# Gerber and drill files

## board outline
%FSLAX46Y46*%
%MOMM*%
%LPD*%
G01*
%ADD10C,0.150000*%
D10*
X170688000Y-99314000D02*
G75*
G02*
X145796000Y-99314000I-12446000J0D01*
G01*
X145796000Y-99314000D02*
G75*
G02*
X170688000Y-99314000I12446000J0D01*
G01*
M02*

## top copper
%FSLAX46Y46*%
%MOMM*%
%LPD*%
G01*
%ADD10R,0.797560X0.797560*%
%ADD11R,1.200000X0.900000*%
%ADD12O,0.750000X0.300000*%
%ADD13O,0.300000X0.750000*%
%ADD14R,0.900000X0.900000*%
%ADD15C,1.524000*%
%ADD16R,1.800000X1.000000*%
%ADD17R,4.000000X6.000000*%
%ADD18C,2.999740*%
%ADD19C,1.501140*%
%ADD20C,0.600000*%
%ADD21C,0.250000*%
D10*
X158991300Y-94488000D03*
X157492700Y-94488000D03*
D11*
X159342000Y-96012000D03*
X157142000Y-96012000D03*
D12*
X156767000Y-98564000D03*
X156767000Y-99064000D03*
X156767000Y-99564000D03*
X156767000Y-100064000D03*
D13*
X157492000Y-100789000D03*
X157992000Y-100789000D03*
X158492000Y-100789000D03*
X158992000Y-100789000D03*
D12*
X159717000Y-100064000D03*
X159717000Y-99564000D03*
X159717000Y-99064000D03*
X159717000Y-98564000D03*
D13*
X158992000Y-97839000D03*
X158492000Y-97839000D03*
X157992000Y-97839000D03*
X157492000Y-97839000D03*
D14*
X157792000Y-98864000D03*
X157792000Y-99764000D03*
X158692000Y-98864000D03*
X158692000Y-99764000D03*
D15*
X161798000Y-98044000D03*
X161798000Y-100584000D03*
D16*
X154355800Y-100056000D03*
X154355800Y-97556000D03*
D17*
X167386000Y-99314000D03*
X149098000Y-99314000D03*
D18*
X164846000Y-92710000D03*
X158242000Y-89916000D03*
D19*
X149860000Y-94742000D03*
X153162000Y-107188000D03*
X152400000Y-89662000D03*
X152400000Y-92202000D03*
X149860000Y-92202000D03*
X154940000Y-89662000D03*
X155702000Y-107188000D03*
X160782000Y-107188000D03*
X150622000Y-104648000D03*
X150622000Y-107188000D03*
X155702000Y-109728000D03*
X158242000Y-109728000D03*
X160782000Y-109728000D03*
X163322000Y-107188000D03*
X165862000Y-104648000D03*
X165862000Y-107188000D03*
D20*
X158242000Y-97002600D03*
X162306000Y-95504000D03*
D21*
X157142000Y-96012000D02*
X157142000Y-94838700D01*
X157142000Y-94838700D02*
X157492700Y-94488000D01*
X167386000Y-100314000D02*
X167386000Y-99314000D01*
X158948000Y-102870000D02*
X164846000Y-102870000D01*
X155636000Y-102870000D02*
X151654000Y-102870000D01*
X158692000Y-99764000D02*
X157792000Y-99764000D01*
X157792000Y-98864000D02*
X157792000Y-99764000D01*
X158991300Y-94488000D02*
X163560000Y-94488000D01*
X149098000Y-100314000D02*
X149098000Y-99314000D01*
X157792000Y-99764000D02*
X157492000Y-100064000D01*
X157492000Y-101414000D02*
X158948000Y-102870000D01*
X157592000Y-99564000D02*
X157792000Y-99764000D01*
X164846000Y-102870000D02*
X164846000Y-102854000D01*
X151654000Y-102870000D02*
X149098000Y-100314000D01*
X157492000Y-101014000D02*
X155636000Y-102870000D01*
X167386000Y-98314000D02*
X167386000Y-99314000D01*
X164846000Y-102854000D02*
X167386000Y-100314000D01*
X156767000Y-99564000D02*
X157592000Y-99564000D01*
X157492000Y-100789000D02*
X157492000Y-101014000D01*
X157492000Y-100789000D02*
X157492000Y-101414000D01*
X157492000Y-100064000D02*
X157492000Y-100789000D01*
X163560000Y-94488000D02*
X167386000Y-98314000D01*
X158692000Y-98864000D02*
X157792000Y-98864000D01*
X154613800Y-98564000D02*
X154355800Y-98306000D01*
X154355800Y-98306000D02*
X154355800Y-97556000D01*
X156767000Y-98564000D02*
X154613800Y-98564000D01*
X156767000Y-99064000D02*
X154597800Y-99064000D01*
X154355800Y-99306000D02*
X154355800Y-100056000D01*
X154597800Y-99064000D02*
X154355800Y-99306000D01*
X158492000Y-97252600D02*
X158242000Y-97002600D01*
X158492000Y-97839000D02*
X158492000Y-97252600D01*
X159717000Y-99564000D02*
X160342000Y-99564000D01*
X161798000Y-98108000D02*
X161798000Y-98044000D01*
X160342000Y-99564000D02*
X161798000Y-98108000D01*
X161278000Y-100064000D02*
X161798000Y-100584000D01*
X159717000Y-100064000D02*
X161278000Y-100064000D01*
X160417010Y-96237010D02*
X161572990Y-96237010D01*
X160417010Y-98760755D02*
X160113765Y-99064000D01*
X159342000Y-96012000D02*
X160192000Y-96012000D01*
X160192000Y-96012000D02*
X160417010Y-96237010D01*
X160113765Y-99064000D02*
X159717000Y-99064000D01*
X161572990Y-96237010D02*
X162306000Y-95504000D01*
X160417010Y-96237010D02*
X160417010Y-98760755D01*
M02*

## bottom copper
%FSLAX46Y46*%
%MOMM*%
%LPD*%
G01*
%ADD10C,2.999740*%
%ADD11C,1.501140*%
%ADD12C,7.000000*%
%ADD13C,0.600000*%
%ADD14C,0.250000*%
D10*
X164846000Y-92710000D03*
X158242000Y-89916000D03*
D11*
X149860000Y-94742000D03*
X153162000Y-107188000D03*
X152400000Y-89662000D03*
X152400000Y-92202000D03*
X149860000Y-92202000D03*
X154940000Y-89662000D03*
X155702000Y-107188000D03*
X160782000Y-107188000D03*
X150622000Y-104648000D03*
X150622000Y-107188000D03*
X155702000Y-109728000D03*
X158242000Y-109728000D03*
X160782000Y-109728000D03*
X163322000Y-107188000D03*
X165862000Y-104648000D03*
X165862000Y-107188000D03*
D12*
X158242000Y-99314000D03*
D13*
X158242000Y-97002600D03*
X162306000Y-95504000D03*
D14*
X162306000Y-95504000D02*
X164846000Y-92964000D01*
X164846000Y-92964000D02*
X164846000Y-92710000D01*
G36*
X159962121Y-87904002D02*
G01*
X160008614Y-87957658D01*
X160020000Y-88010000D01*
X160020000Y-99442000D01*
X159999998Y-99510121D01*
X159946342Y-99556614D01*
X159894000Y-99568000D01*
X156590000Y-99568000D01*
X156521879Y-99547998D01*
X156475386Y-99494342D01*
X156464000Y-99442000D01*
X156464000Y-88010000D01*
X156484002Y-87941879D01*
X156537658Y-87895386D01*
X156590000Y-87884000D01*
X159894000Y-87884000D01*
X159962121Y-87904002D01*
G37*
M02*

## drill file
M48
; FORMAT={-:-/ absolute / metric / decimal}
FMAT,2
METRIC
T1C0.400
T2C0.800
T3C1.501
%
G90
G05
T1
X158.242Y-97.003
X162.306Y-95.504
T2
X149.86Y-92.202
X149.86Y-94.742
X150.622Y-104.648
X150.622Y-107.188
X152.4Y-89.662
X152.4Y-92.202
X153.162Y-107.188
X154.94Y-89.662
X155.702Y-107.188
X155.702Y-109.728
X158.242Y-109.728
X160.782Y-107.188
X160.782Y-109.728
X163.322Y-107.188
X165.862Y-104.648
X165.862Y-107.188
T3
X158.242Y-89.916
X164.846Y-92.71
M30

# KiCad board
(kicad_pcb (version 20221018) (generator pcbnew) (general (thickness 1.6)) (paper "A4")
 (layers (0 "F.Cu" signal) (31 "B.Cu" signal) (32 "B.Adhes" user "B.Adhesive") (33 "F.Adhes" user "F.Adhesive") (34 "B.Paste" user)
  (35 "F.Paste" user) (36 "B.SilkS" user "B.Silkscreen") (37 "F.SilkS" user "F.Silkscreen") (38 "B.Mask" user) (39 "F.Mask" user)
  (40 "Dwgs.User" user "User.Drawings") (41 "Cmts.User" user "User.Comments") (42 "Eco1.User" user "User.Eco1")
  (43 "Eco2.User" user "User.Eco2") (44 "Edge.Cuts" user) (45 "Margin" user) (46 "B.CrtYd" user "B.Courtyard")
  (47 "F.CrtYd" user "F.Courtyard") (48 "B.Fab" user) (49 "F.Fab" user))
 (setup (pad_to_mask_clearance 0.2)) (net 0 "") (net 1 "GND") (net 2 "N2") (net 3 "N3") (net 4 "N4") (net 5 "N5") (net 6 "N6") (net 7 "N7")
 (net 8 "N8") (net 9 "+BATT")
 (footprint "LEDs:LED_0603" (layer "F.Cu") (at 158.242 94.488 180)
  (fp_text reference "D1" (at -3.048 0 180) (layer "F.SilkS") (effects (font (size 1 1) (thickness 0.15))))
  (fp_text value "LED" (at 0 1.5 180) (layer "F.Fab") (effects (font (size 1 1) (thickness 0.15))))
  (pad "1" smd rect (at -0.7493 0) (size 0.79756 0.79756) (layers "F.Cu" "F.Paste" "F.Mask") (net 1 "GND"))
  (pad "2" smd rect (at 0.7493 0) (size 0.79756 0.79756) (layers "F.Cu" "F.Paste" "F.Mask") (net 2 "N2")))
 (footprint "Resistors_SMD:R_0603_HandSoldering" (layer "F.Cu") (at 158.242 96.012 180)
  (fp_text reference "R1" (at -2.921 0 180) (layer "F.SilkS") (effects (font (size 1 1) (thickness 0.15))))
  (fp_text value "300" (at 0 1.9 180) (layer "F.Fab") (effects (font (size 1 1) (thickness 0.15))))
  (pad "1" smd rect (at -1.1 0 180) (size 1.2 0.9) (layers "F.Cu" "F.Paste" "F.Mask") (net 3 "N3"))
  (pad "2" smd rect (at 1.1 0 180) (size 1.2 0.9) (layers "F.Cu" "F.Paste" "F.Mask") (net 2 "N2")))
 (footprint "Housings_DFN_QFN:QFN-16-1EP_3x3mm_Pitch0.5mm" (layer "F.Cu") (at 158.242 99.314)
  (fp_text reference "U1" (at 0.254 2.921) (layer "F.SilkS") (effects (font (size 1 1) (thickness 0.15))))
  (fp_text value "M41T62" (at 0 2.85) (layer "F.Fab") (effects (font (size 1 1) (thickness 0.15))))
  (pad "1" smd oval (at -1.475 -0.75) (size 0.75 0.3) (layers "F.Cu" "F.Paste" "F.Mask") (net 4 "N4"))
  (pad "2" smd oval (at -1.475 -0.25) (size 0.75 0.3) (layers "F.Cu" "F.Paste" "F.Mask") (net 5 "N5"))
  (pad "3" smd oval (at -1.475 0.25) (size 0.75 0.3) (layers "F.Cu" "F.Paste" "F.Mask") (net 1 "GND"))
  (pad "4" smd oval (at -1.475 0.75) (size 0.75 0.3) (layers "F.Cu" "F.Paste" "F.Mask") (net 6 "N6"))
  (pad "5" smd oval (at -0.75 1.475 90) (size 0.75 0.3) (layers "F.Cu" "F.Paste" "F.Mask") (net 1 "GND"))
  (pad "6" smd oval (at -0.25 1.475 90) (size 0.75 0.3) (layers "F.Cu" "F.Paste" "F.Mask"))
  (pad "7" smd oval (at 0.25 1.475 90) (size 0.75 0.3) (layers "F.Cu" "F.Paste" "F.Mask"))
  (pad "8" smd oval (at 0.75 1.475 90) (size 0.75 0.3) (layers "F.Cu" "F.Paste" "F.Mask"))
  (pad "9" smd oval (at 1.475 0.75) (size 0.75 0.3) (layers "F.Cu" "F.Paste" "F.Mask") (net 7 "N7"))
  (pad "10" smd oval (at 1.475 0.25) (size 0.75 0.3) (layers "F.Cu" "F.Paste" "F.Mask") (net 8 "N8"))
  (pad "11" smd oval (at 1.475 -0.25) (size 0.75 0.3) (layers "F.Cu" "F.Paste" "F.Mask") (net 3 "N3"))
  (pad "12" smd oval (at 1.475 -0.75) (size 0.75 0.3) (layers "F.Cu" "F.Paste" "F.Mask"))
  (pad "13" smd oval (at 0.75 -1.475 90) (size 0.75 0.3) (layers "F.Cu" "F.Paste" "F.Mask"))
  (pad "14" smd oval (at 0.25 -1.475 90) (size 0.75 0.3) (layers "F.Cu" "F.Paste" "F.Mask") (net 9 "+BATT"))
  (pad "15" smd oval (at -0.25 -1.475 90) (size 0.75 0.3) (layers "F.Cu" "F.Paste" "F.Mask"))
  (pad "16" smd oval (at -0.75 -1.475 90) (size 0.75 0.3) (layers "F.Cu" "F.Paste" "F.Mask"))
  (pad "17" smd rect (at -0.45 -0.45) (size 0.9 0.9) (layers "F.Cu" "F.Paste" "F.Mask") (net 1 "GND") (solder_paste_margin_ratio -0.2))
  (pad "17" smd rect (at -0.45 0.45) (size 0.9 0.9) (layers "F.Cu" "F.Paste" "F.Mask") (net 1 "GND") (solder_paste_margin_ratio -0.2))
  (pad "17" smd rect (at 0.45 -0.45) (size 0.9 0.9) (layers "F.Cu" "F.Paste" "F.Mask") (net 1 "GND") (solder_paste_margin_ratio -0.2))
  (pad "17" smd rect (at 0.45 0.45) (size 0.9 0.9) (layers "F.Cu" "F.Paste" "F.Mask") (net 1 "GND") (solder_paste_margin_ratio -0.2)))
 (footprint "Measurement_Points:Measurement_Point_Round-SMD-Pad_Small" (layer "F.Cu") (at 161.798 98.044)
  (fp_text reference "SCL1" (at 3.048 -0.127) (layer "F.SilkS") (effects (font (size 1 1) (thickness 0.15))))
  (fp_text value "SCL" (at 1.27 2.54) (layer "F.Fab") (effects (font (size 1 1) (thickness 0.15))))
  (pad "1" smd circle (at 0 0) (size 1.524 1.524) (layers "F.Cu" "F.Mask") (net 8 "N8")))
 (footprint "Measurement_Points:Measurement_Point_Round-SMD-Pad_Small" (layer "F.Cu") (at 161.798 100.584)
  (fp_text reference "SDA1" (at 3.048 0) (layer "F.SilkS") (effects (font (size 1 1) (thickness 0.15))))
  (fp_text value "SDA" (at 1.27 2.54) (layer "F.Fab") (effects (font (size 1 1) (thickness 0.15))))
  (pad "1" smd circle (at 0 0) (size 1.524 1.524) (layers "F.Cu" "F.Mask") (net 7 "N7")))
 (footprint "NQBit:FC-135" (layer "F.Cu") (at 154.3558 98.806 -90)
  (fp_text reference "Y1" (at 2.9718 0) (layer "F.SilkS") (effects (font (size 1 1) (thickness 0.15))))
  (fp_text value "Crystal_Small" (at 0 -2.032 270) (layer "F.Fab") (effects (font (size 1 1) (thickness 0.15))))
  (pad "1" smd rect (at 1.25 0 270) (size 1 1.8) (layers "F.Cu" "F.Paste" "F.Mask") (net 5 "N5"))
  (pad "2" smd rect (at -1.25 0 270) (size 1 1.8) (layers "F.Cu" "F.Paste" "F.Mask") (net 4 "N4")))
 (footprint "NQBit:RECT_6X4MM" (layer "F.Cu") (at 167.386 99.314)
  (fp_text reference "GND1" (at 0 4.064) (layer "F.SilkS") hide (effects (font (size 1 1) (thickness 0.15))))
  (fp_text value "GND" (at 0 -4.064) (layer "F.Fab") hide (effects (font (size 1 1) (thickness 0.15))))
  (pad "1" smd rect (at 0 0) (size 4 6) (layers "F.Cu" "F.Paste" "F.Mask") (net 1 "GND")))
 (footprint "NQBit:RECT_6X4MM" (layer "F.Cu") (at 149.098 99.314)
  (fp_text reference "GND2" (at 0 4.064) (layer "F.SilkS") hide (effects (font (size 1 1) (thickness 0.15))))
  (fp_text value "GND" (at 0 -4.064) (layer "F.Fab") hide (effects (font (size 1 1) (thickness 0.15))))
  (pad "1" smd rect (at 0 0) (size 4 6) (layers "F.Cu" "F.Paste" "F.Mask") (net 1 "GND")))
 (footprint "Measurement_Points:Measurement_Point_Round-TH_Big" (layer "F.Cu") (at 164.846 92.71)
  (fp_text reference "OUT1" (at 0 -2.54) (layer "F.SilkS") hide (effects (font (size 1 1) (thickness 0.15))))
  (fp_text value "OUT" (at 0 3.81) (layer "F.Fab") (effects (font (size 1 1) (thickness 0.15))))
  (pad "1" thru_hole circle (at 0 0) (size 2.99974 2.99974) (drill 1.50114) (layers "*.Cu" "*.Mask" "F.SilkS") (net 3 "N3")))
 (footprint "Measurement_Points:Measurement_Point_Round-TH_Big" (layer "F.Cu") (at 158.242 89.916)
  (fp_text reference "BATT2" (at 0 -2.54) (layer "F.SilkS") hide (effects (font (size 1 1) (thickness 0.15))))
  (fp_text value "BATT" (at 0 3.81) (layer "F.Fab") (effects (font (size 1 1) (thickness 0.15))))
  (pad "1" thru_hole circle (at 0 0) (size 2.99974 2.99974) (drill 1.50114) (layers "*.Cu" "*.Mask" "F.SilkS") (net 9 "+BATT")))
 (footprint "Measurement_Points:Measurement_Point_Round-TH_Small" (layer "F.Cu") (at 149.86 94.742)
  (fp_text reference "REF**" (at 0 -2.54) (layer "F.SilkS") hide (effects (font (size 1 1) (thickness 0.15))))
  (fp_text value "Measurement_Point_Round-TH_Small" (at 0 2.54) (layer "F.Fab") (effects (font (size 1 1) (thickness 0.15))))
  (pad "1" thru_hole circle (at 0 0) (size 1.50114 1.50114) (drill 0.8001) (layers "*.Cu" "*.Mask" "F.SilkS")))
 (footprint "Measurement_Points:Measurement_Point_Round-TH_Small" (layer "F.Cu") (at 153.162 107.188)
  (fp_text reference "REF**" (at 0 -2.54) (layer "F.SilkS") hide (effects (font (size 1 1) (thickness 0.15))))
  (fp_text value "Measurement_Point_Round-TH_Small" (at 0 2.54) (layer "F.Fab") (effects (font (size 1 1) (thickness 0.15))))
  (pad "1" thru_hole circle (at 0 0) (size 1.50114 1.50114) (drill 0.8001) (layers "*.Cu" "*.Mask" "F.SilkS")))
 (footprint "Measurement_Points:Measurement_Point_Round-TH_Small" (layer "F.Cu") (at 152.4 89.662)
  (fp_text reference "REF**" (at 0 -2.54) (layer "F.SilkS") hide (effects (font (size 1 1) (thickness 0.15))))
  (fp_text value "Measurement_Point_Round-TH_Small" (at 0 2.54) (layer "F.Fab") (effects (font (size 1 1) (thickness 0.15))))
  (pad "1" thru_hole circle (at 0 0) (size 1.50114 1.50114) (drill 0.8001) (layers "*.Cu" "*.Mask" "F.SilkS")))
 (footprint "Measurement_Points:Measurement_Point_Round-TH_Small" (layer "F.Cu") (at 152.4 92.202)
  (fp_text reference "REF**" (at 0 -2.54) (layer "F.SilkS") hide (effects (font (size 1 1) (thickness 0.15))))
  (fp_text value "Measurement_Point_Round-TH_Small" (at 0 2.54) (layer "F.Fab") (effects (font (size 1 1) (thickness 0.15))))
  (pad "1" thru_hole circle (at 0 0) (size 1.50114 1.50114) (drill 0.8001) (layers "*.Cu" "*.Mask" "F.SilkS")))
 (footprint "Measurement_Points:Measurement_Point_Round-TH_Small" (layer "F.Cu") (at 149.86 92.202)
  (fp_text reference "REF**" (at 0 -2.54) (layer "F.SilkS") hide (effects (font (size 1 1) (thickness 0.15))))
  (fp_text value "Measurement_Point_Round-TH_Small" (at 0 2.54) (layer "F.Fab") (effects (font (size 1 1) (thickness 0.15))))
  (pad "1" thru_hole circle (at 0 0) (size 1.50114 1.50114) (drill 0.8001) (layers "*.Cu" "*.Mask" "F.SilkS")))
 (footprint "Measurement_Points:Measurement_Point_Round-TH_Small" (layer "F.Cu") (at 154.94 89.662)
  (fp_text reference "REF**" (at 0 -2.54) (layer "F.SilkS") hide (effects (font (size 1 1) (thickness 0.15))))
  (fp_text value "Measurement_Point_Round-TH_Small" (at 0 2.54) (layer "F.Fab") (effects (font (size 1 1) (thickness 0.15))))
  (pad "1" thru_hole circle (at 0 0) (size 1.50114 1.50114) (drill 0.8001) (layers "*.Cu" "*.Mask" "F.SilkS")))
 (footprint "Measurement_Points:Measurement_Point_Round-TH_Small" (layer "F.Cu") (at 155.702 107.188)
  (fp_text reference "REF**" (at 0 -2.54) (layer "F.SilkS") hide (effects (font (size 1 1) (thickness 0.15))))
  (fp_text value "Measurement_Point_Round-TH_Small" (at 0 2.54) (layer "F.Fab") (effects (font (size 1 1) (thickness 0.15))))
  (pad "1" thru_hole circle (at 0 0) (size 1.50114 1.50114) (drill 0.8001) (layers "*.Cu" "*.Mask" "F.SilkS")))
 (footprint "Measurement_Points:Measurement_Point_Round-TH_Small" (layer "F.Cu") (at 160.782 107.188)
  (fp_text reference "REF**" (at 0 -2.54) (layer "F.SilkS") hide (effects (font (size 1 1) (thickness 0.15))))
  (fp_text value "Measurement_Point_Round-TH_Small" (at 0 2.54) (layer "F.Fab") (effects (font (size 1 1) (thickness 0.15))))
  (pad "1" thru_hole circle (at 0 0) (size 1.50114 1.50114) (drill 0.8001) (layers "*.Cu" "*.Mask" "F.SilkS")))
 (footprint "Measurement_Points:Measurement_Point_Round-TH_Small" (layer "F.Cu") (at 150.622 104.648)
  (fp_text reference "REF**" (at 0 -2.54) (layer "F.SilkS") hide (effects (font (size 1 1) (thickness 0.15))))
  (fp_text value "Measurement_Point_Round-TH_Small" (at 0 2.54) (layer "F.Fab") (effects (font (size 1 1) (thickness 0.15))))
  (pad "1" thru_hole circle (at 0 0) (size 1.50114 1.50114) (drill 0.8001) (layers "*.Cu" "*.Mask" "F.SilkS")))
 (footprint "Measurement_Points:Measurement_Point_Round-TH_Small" (layer "F.Cu") (at 150.622 107.188)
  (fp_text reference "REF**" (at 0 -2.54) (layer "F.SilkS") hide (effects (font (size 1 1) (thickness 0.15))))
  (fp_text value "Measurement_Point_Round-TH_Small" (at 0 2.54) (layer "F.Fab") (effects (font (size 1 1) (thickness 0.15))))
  (pad "1" thru_hole circle (at 0 0) (size 1.50114 1.50114) (drill 0.8001) (layers "*.Cu" "*.Mask" "F.SilkS")))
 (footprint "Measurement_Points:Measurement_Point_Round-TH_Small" (layer "F.Cu") (at 155.702 109.728)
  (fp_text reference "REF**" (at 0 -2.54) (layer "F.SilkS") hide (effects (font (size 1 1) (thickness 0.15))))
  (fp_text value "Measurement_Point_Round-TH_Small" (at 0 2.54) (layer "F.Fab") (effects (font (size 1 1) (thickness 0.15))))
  (pad "1" thru_hole circle (at 0 0) (size 1.50114 1.50114) (drill 0.8001) (layers "*.Cu" "*.Mask" "F.SilkS")))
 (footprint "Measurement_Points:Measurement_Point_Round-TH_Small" (layer "F.Cu") (at 158.242 109.728)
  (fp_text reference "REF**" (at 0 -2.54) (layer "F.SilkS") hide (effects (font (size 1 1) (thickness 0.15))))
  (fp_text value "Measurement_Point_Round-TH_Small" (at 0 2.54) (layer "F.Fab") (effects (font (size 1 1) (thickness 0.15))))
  (pad "1" thru_hole circle (at 0 0) (size 1.50114 1.50114) (drill 0.8001) (layers "*.Cu" "*.Mask" "F.SilkS")))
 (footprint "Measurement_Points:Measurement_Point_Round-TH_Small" (layer "F.Cu") (at 160.782 109.728)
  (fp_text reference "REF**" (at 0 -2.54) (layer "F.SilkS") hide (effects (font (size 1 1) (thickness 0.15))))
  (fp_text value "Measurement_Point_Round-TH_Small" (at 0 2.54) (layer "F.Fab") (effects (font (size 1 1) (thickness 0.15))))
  (pad "1" thru_hole circle (at 0 0) (size 1.50114 1.50114) (drill 0.8001) (layers "*.Cu" "*.Mask" "F.SilkS")))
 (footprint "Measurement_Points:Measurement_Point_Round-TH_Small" (layer "F.Cu") (at 163.322 107.188)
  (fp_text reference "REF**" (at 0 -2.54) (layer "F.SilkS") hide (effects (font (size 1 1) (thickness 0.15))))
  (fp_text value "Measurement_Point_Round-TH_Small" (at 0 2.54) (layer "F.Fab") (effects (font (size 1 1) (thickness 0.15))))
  (pad "1" thru_hole circle (at 0 0) (size 1.50114 1.50114) (drill 0.8001) (layers "*.Cu" "*.Mask" "F.SilkS")))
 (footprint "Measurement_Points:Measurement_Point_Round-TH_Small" (layer "F.Cu") (at 165.862 104.648)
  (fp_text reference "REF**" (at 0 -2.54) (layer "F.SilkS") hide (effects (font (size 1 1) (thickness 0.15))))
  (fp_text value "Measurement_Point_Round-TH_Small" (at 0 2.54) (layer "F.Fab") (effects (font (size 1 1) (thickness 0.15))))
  (pad "1" thru_hole circle (at 0 0) (size 1.50114 1.50114) (drill 0.8001) (layers "*.Cu" "*.Mask" "F.SilkS")))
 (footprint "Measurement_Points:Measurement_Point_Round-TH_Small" (layer "F.Cu") (at 165.862 107.188)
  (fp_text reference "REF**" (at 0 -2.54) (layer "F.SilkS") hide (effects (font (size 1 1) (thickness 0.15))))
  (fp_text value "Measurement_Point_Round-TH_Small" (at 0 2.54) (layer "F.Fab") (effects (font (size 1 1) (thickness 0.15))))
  (pad "1" thru_hole circle (at 0 0) (size 1.50114 1.50114) (drill 0.8001) (layers "*.Cu" "*.Mask" "F.SilkS")))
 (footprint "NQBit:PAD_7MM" (layer "B.Cu") (at 158.242 99.314)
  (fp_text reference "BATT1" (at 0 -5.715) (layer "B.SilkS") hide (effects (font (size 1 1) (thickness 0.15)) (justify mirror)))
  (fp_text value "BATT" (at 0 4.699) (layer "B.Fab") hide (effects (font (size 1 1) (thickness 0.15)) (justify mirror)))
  (pad "1" smd circle (at 0 0) (size 7 7) (layers "B.Cu" "B.Paste" "B.Mask") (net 9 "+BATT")))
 (gr_circle (center 158.242 99.314) (end 158.242 86.868) (stroke (width 0.15) (type solid)) (fill none) (layer "Edge.Cuts"))
 (segment (start 157.142 96.012) (end 157.142 94.8387) (width 0.25) (layer "F.Cu") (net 2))
 (segment (start 157.142 94.8387) (end 157.4927 94.488) (width 0.25) (layer "F.Cu") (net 2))
 (segment (start 167.386 100.314) (end 167.386 99.314) (width 0.25) (layer "F.Cu") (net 1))
 (segment (start 158.948 102.87) (end 164.846 102.87) (width 0.25) (layer "F.Cu") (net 1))
 (segment (start 155.636 102.87) (end 151.654 102.87) (width 0.25) (layer "F.Cu") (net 1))
 (segment (start 158.692 99.764) (end 157.792 99.764) (width 0.25) (layer "F.Cu") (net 1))
 (segment (start 157.792 98.864) (end 157.792 99.764) (width 0.25) (layer "F.Cu") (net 1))
 (segment (start 158.9913 94.488) (end 163.56 94.488) (width 0.25) (layer "F.Cu") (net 1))
 (segment (start 149.098 100.314) (end 149.098 99.314) (width 0.25) (layer "F.Cu") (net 1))
 (segment (start 157.792 99.764) (end 157.492 100.064) (width 0.25) (layer "F.Cu") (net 1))
 (segment (start 157.492 101.414) (end 158.948 102.87) (width 0.25) (layer "F.Cu") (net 1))
 (segment (start 157.592 99.564) (end 157.792 99.764) (width 0.25) (layer "F.Cu") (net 1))
 (segment (start 164.846 102.87) (end 164.846 102.854) (width 0.25) (layer "F.Cu") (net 1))
 (segment (start 151.654 102.87) (end 149.098 100.314) (width 0.25) (layer "F.Cu") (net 1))
 (segment (start 157.492 101.014) (end 155.636 102.87) (width 0.25) (layer "F.Cu") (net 1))
 (segment (start 167.386 98.314) (end 167.386 99.314) (width 0.25) (layer "F.Cu") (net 1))
 (segment (start 164.846 102.854) (end 167.386 100.314) (width 0.25) (layer "F.Cu") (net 1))
 (segment (start 156.767 99.564) (end 157.592 99.564) (width 0.25) (layer "F.Cu") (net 1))
 (segment (start 157.492 100.789) (end 157.492 101.014) (width 0.25) (layer "F.Cu") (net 1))
 (segment (start 157.492 100.789) (end 157.492 101.414) (width 0.25) (layer "F.Cu") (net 1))
 (segment (start 157.492 100.064) (end 157.492 100.789) (width 0.25) (layer "F.Cu") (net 1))
 (segment (start 163.56 94.488) (end 167.386 98.314) (width 0.25) (layer "F.Cu") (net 1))
 (segment (start 158.692 98.864) (end 157.792 98.864) (width 0.25) (layer "F.Cu") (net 1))
 (segment (start 154.6138 98.564) (end 154.3558 98.306) (width 0.25) (layer "F.Cu") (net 4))
 (segment (start 154.3558 98.306) (end 154.3558 97.556) (width 0.25) (layer "F.Cu") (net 4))
 (segment (start 156.767 98.564) (end 154.6138 98.564) (width 0.25) (layer "F.Cu") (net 4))
 (segment (start 156.767 99.064) (end 154.5978 99.064) (width 0.25) (layer "F.Cu") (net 5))
 (segment (start 154.3558 99.306) (end 154.3558 100.056) (width 0.25) (layer "F.Cu") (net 5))
 (segment (start 154.5978 99.064) (end 154.3558 99.306) (width 0.25) (layer "F.Cu") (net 5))
 (segment (start 158.492 97.2526) (end 158.242 97.0026) (width 0.25) (layer "F.Cu") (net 9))
 (segment (start 158.492 97.839) (end 158.492 97.2526) (width 0.25) (layer "F.Cu") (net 9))
 (via (at 158.242 97.0026) (size 0.6) (drill 0.4) (layers "F.Cu" "B.Cu") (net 9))
 (segment (start 159.717 99.564) (end 160.342 99.564) (width 0.25) (layer "F.Cu") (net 8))
 (segment (start 161.798 98.108) (end 161.798 98.044) (width 0.25) (layer "F.Cu") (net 8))
 (segment (start 160.342 99.564) (end 161.798 98.108) (width 0.25) (layer "F.Cu") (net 8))
 (segment (start 161.278 100.064) (end 161.798 100.584) (width 0.25) (layer "F.Cu") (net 7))
 (segment (start 159.717 100.064) (end 161.278 100.064) (width 0.25) (layer "F.Cu") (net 7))
 (segment (start 160.41701 96.23701) (end 161.57299 96.23701) (width 0.25) (layer "F.Cu") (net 3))
 (segment (start 160.41701 98.760755) (end 160.113765 99.064) (width 0.25) (layer "F.Cu") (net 3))
 (segment (start 159.342 96.012) (end 160.192 96.012) (width 0.25) (layer "F.Cu") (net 3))
 (segment (start 160.192 96.012) (end 160.41701 96.23701) (width 0.25) (layer "F.Cu") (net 3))
 (segment (start 160.113765 99.064) (end 159.717 99.064) (width 0.25) (layer "F.Cu") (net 3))
 (segment (start 161.57299 96.23701) (end 162.306 95.504) (width 0.25) (layer "F.Cu") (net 3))
 (segment (start 160.41701 96.23701) (end 160.41701 98.760755) (width 0.25) (layer "F.Cu") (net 3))
 (via (at 162.306 95.504) (size 0.6) (drill 0.4) (layers "F.Cu" "B.Cu") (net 3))
 (segment (start 162.306 95.504) (end 164.846 92.964) (width 0.25) (layer "B.Cu") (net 3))
 (segment (start 164.846 92.964) (end 164.846 92.71) (width 0.25) (layer "B.Cu") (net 3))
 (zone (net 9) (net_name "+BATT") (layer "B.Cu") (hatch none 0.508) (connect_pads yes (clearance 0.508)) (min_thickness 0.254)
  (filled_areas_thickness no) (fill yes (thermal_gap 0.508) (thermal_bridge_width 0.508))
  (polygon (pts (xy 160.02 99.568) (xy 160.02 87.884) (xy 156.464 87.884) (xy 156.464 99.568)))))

